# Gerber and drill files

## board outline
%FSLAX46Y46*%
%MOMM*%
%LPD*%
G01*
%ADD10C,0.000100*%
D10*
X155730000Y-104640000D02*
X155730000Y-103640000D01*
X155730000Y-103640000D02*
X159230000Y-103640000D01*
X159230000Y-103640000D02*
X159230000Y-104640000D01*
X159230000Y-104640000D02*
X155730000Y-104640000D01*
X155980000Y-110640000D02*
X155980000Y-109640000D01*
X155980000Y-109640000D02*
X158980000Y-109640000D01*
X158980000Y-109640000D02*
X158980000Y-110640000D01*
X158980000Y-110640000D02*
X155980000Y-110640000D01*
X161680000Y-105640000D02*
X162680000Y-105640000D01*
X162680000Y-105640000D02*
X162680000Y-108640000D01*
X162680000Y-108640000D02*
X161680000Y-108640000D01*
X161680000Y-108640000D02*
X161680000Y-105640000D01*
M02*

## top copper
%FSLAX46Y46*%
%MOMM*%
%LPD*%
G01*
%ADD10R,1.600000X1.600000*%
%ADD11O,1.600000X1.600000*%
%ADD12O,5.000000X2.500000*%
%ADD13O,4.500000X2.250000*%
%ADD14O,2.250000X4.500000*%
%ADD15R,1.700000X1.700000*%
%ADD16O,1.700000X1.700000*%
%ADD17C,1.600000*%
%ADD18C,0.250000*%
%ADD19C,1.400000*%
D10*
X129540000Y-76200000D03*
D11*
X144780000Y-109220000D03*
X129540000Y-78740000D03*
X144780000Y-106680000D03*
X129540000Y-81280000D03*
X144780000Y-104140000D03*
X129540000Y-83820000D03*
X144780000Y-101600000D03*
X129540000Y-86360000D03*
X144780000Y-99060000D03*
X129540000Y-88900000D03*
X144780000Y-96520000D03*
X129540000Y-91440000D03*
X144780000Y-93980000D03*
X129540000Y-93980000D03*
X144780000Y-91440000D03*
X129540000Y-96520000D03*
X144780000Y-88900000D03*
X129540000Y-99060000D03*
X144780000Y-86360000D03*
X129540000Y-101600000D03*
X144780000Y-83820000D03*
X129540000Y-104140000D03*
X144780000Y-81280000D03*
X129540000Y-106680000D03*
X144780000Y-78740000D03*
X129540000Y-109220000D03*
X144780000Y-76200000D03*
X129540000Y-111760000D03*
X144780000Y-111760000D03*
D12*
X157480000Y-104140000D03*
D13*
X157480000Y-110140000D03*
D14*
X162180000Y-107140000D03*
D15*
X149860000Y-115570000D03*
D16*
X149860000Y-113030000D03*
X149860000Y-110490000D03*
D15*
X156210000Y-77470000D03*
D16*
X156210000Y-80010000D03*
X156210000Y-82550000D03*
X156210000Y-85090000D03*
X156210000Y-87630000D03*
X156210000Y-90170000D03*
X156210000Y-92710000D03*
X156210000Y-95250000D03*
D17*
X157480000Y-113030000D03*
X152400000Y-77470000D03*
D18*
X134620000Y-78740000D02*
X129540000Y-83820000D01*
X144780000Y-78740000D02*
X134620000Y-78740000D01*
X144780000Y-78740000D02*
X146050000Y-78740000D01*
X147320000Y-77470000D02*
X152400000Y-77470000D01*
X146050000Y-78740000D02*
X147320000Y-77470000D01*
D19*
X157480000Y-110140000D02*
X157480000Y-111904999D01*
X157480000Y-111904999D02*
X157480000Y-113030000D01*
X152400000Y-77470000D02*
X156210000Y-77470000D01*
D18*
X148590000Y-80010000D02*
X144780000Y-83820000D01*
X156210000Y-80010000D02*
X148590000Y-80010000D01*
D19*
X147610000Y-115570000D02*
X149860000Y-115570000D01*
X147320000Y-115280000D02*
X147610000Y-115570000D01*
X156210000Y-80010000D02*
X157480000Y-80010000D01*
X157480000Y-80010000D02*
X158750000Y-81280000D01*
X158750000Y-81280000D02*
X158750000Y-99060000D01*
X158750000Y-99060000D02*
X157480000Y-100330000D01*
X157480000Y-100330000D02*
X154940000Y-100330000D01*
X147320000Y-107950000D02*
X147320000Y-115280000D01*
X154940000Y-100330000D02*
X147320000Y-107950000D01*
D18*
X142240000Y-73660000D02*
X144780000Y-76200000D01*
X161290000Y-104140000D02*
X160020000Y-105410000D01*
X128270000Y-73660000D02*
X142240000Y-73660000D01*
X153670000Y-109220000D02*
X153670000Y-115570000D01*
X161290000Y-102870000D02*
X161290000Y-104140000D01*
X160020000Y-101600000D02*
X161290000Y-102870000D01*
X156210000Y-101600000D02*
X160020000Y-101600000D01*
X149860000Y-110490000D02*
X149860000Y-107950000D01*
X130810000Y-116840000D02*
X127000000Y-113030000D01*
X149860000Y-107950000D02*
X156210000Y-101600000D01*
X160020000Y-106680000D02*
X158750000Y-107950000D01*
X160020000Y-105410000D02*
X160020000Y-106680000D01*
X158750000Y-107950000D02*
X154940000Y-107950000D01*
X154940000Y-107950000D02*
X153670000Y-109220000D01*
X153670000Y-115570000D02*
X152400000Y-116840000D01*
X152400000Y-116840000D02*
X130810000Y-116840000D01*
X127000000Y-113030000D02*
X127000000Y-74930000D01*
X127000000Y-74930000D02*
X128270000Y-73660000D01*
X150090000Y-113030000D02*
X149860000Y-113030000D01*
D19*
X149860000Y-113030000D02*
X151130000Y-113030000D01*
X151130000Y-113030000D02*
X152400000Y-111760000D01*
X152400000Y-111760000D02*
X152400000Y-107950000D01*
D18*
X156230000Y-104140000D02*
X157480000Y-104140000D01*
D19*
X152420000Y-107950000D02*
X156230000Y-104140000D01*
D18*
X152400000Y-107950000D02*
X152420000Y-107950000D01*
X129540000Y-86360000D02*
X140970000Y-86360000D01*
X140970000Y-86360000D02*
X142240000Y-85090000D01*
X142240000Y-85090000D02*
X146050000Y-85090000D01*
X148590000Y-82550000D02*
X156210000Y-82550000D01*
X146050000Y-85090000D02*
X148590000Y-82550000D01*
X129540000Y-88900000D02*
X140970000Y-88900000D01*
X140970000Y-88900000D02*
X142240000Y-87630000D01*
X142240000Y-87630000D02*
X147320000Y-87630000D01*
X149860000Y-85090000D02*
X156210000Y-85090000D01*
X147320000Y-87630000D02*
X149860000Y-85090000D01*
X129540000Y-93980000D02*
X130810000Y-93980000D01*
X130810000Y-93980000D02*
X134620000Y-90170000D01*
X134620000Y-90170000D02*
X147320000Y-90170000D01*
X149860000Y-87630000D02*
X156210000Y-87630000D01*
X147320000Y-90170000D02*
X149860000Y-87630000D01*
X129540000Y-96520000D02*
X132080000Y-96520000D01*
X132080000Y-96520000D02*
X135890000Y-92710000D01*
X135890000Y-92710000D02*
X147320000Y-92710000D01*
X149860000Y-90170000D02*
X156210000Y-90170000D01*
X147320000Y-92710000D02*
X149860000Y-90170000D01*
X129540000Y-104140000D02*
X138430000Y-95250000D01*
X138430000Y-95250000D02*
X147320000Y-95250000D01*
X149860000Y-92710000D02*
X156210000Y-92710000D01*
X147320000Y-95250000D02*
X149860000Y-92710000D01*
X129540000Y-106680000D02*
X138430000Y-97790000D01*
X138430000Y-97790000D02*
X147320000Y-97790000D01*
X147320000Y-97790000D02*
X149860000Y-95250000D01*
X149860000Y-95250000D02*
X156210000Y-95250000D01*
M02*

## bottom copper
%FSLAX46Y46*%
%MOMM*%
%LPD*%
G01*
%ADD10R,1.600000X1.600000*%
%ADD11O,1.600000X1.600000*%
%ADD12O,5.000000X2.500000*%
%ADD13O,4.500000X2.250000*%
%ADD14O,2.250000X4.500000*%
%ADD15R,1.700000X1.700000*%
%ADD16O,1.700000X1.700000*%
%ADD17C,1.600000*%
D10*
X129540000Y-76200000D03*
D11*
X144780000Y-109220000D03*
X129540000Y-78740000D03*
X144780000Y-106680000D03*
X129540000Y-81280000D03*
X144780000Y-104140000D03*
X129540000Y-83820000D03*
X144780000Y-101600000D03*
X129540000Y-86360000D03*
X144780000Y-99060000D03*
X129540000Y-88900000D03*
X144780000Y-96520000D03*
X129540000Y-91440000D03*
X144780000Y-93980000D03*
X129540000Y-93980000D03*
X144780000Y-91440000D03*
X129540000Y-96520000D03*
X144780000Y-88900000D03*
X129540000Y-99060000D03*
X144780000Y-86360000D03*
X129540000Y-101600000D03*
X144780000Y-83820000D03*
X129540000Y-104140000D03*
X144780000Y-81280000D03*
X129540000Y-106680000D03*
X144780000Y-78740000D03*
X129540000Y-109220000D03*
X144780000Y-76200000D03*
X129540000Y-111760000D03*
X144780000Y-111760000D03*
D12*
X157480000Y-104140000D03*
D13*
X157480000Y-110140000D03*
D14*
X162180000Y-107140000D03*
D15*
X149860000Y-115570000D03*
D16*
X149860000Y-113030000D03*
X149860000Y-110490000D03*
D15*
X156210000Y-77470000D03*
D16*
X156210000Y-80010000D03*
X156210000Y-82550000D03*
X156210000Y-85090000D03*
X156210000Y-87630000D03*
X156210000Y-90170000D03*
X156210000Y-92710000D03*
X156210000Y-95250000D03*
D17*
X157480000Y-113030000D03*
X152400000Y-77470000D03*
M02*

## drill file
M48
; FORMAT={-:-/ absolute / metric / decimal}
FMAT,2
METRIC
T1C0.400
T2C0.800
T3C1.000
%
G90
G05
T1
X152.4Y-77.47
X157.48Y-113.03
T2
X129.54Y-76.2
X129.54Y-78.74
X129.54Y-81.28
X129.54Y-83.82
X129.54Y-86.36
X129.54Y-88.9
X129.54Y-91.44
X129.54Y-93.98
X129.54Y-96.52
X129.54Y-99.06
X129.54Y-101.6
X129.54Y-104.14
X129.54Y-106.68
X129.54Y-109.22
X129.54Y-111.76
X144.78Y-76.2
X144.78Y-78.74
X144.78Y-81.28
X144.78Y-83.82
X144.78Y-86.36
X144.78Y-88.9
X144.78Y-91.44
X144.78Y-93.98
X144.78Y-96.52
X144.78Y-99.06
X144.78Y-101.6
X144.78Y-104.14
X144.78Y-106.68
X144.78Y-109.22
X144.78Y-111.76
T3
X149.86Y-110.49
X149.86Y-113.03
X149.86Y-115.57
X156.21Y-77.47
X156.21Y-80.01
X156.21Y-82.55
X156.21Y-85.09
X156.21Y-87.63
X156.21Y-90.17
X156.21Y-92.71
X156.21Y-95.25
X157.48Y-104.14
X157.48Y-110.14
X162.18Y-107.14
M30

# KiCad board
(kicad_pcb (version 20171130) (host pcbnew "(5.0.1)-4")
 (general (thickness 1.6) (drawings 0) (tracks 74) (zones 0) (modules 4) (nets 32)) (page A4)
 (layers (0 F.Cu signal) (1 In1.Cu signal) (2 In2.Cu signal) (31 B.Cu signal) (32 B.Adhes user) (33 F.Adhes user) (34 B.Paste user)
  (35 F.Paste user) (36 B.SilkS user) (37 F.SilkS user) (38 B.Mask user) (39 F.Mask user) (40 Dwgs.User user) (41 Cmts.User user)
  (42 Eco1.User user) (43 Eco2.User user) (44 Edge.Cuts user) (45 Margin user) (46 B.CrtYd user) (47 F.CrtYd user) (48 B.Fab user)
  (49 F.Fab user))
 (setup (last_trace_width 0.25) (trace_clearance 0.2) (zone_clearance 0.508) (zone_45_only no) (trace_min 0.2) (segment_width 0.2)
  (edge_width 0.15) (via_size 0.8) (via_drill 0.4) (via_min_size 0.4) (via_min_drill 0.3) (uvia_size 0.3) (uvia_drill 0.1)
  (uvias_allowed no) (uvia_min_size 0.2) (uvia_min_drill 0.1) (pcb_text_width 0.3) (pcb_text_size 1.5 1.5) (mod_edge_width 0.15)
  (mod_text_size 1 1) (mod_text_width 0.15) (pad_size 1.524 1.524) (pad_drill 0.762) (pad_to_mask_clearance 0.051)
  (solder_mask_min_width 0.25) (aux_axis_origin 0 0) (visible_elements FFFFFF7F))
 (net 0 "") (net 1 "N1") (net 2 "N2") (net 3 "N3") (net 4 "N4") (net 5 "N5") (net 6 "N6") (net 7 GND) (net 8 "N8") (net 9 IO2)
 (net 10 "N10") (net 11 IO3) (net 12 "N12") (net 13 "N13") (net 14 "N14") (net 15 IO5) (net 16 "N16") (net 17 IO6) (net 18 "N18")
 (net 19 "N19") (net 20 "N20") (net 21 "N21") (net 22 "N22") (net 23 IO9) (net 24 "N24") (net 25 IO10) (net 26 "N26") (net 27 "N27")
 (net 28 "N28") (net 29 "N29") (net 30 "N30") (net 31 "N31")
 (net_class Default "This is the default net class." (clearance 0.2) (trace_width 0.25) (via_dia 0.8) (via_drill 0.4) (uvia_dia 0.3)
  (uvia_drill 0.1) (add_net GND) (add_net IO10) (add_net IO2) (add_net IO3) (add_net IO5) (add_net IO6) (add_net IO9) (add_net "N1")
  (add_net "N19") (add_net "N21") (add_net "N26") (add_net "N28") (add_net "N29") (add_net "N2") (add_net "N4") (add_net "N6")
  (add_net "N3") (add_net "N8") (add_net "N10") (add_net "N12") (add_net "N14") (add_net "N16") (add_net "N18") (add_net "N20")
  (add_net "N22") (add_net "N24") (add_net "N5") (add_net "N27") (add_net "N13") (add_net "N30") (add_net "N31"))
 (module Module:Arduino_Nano (layer F.Cu) (at 129.54 76.2)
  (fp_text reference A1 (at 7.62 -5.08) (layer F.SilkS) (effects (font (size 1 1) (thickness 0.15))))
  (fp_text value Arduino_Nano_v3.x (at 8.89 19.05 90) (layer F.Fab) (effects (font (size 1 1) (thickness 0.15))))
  (pad 1 thru_hole rect (at 0 0) (size 1.6 1.6) (drill 0.8) (layers *.Cu *.Mask) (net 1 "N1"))
  (pad 17 thru_hole oval (at 15.24 33.02) (size 1.6 1.6) (drill 0.8) (layers *.Cu *.Mask) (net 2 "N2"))
  (pad 2 thru_hole oval (at 0 2.54) (size 1.6 1.6) (drill 0.8) (layers *.Cu *.Mask) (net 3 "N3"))
  (pad 18 thru_hole oval (at 15.24 30.48) (size 1.6 1.6) (drill 0.8) (layers *.Cu *.Mask) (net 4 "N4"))
  (pad 3 thru_hole oval (at 0 5.08) (size 1.6 1.6) (drill 0.8) (layers *.Cu *.Mask) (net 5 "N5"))
  (pad 19 thru_hole oval (at 15.24 27.94) (size 1.6 1.6) (drill 0.8) (layers *.Cu *.Mask) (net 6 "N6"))
  (pad 4 thru_hole oval (at 0 7.62) (size 1.6 1.6) (drill 0.8) (layers *.Cu *.Mask) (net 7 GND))
  (pad 20 thru_hole oval (at 15.24 25.4) (size 1.6 1.6) (drill 0.8) (layers *.Cu *.Mask) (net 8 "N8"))
  (pad 5 thru_hole oval (at 0 10.16) (size 1.6 1.6) (drill 0.8) (layers *.Cu *.Mask) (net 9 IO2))
  (pad 21 thru_hole oval (at 15.24 22.86) (size 1.6 1.6) (drill 0.8) (layers *.Cu *.Mask) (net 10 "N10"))
  (pad 6 thru_hole oval (at 0 12.7) (size 1.6 1.6) (drill 0.8) (layers *.Cu *.Mask) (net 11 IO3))
  (pad 22 thru_hole oval (at 15.24 20.32) (size 1.6 1.6) (drill 0.8) (layers *.Cu *.Mask) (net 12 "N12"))
  (pad 7 thru_hole oval (at 0 15.24) (size 1.6 1.6) (drill 0.8) (layers *.Cu *.Mask) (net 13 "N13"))
  (pad 23 thru_hole oval (at 15.24 17.78) (size 1.6 1.6) (drill 0.8) (layers *.Cu *.Mask) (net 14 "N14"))
  (pad 8 thru_hole oval (at 0 17.78) (size 1.6 1.6) (drill 0.8) (layers *.Cu *.Mask) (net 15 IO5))
  (pad 24 thru_hole oval (at 15.24 15.24) (size 1.6 1.6) (drill 0.8) (layers *.Cu *.Mask) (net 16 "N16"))
  (pad 9 thru_hole oval (at 0 20.32) (size 1.6 1.6) (drill 0.8) (layers *.Cu *.Mask) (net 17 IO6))
  (pad 25 thru_hole oval (at 15.24 12.7) (size 1.6 1.6) (drill 0.8) (layers *.Cu *.Mask) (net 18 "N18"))
  (pad 10 thru_hole oval (at 0 22.86) (size 1.6 1.6) (drill 0.8) (layers *.Cu *.Mask) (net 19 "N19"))
  (pad 26 thru_hole oval (at 15.24 10.16) (size 1.6 1.6) (drill 0.8) (layers *.Cu *.Mask) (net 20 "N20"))
  (pad 11 thru_hole oval (at 0 25.4) (size 1.6 1.6) (drill 0.8) (layers *.Cu *.Mask) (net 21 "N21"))
  (pad 27 thru_hole oval (at 15.24 7.62) (size 1.6 1.6) (drill 0.8) (layers *.Cu *.Mask) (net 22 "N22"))
  (pad 12 thru_hole oval (at 0 27.94) (size 1.6 1.6) (drill 0.8) (layers *.Cu *.Mask) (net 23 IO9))
  (pad 28 thru_hole oval (at 15.24 5.08) (size 1.6 1.6) (drill 0.8) (layers *.Cu *.Mask) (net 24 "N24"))
  (pad 13 thru_hole oval (at 0 30.48) (size 1.6 1.6) (drill 0.8) (layers *.Cu *.Mask) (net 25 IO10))
  (pad 29 thru_hole oval (at 15.24 2.54) (size 1.6 1.6) (drill 0.8) (layers *.Cu *.Mask) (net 7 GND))
  (pad 14 thru_hole oval (at 0 33.02) (size 1.6 1.6) (drill 0.8) (layers *.Cu *.Mask) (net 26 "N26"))
  (pad 30 thru_hole oval (at 15.24 0) (size 1.6 1.6) (drill 0.8) (layers *.Cu *.Mask) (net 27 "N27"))
  (pad 15 thru_hole oval (at 0 35.56) (size 1.6 1.6) (drill 0.8) (layers *.Cu *.Mask) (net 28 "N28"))
  (pad 16 thru_hole oval (at 15.24 35.56) (size 1.6 1.6) (drill 0.8) (layers *.Cu *.Mask) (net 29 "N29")))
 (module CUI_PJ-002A (layer F.Cu) (at 157.48 104.14 270)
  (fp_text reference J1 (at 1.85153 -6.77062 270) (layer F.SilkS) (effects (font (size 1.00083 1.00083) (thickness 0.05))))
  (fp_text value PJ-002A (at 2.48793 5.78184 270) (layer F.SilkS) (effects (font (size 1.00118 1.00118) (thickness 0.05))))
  (fp_line (start 0.5 1.75) (end -0.5 1.75) (layer Edge.Cuts) (width 0.0001))
  (fp_line (start -0.5 1.75) (end -0.5 -1.75) (layer Edge.Cuts) (width 0.0001))
  (fp_line (start -0.5 -1.75) (end 0.5 -1.75) (layer Edge.Cuts) (width 0.0001))
  (fp_line (start 0.5 -1.75) (end 0.5 1.75) (layer Edge.Cuts) (width 0.0001))
  (fp_line (start 6.5 1.5) (end 5.5 1.5) (layer Edge.Cuts) (width 0.0001))
  (fp_line (start 5.5 1.5) (end 5.5 -1.5) (layer Edge.Cuts) (width 0.0001))
  (fp_line (start 5.5 -1.5) (end 6.5 -1.5) (layer Edge.Cuts) (width 0.0001))
  (fp_line (start 6.5 -1.5) (end 6.5 1.5) (layer Edge.Cuts) (width 0.0001))
  (fp_line (start 1.5 -4.2) (end 1.5 -5.2) (layer Edge.Cuts) (width 0.0001))
  (fp_line (start 1.5 -5.2) (end 4.5 -5.2) (layer Edge.Cuts) (width 0.0001))
  (fp_line (start 4.5 -5.2) (end 4.5 -4.2) (layer Edge.Cuts) (width 0.0001))
  (fp_line (start 4.5 -4.2) (end 1.5 -4.2) (layer Edge.Cuts) (width 0.0001))
  (pad 1 thru_hole oval (at 0 0) (size 5 2.5) (drill 1) (layers *.Cu *.Mask) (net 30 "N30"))
  (pad 2 thru_hole oval (at 6 0) (size 4.5 2.25) (drill 1) (layers *.Cu *.Mask) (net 7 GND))
  (pad 3 thru_hole oval (at 3 -4.7 90) (size 4.5 2.25) (drill 1) (layers *.Cu *.Mask) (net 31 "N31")))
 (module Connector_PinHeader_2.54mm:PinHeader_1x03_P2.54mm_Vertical (layer F.Cu) (at 149.86 115.57 180)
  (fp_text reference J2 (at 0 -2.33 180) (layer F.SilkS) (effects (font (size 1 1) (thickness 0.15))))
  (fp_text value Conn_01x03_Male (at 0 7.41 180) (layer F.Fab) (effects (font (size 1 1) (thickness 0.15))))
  (pad 1 thru_hole rect (at 0 0 180) (size 1.7 1.7) (drill 1) (layers *.Cu *.Mask) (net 22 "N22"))
  (pad 2 thru_hole oval (at 0 2.54 180) (size 1.7 1.7) (drill 1) (layers *.Cu *.Mask) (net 30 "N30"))
  (pad 3 thru_hole oval (at 0 5.08 180) (size 1.7 1.7) (drill 1) (layers *.Cu *.Mask) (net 27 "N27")))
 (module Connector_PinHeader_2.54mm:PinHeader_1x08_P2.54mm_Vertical (layer F.Cu) (at 156.21 77.47)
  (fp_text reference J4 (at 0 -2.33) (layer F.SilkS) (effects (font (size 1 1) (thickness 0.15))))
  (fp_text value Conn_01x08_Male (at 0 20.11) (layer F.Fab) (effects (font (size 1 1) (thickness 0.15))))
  (pad 1 thru_hole rect (at 0 0) (size 1.7 1.7) (drill 1) (layers *.Cu *.Mask) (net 7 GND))
  (pad 2 thru_hole oval (at 0 2.54) (size 1.7 1.7) (drill 1) (layers *.Cu *.Mask) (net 22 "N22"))
  (pad 3 thru_hole oval (at 0 5.08) (size 1.7 1.7) (drill 1) (layers *.Cu *.Mask) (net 9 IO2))
  (pad 4 thru_hole oval (at 0 7.62) (size 1.7 1.7) (drill 1) (layers *.Cu *.Mask) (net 11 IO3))
  (pad 5 thru_hole oval (at 0 10.16) (size 1.7 1.7) (drill 1) (layers *.Cu *.Mask) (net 15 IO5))
  (pad 6 thru_hole oval (at 0 12.7) (size 1.7 1.7) (drill 1) (layers *.Cu *.Mask) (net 17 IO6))
  (pad 7 thru_hole oval (at 0 15.24) (size 1.7 1.7) (drill 1) (layers *.Cu *.Mask) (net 23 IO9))
  (pad 8 thru_hole oval (at 0 17.78) (size 1.7 1.7) (drill 1) (layers *.Cu *.Mask) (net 25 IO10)))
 (via (at 157.48 113.03) (size 1.6) (drill 0.4) (layers F.Cu B.Cu) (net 7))
 (segment (start 134.62 78.74) (end 129.54 83.82) (width 0.25) (layer F.Cu) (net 7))
 (segment (start 144.78 78.74) (end 134.62 78.74) (width 0.25) (layer F.Cu) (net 7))
 (segment (start 144.78 78.74) (end 146.05 78.74) (width 0.25) (layer F.Cu) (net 7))
 (segment (start 147.32 77.47) (end 152.4 77.47) (width 0.25) (layer F.Cu) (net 7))
 (segment (start 146.05 78.74) (end 147.32 77.47) (width 0.25) (layer F.Cu) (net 7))
 (segment (start 157.48 110.14) (end 157.48 111.904999) (width 1.4) (layer F.Cu) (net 7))
 (segment (start 157.48 111.904999) (end 157.48 113.03) (width 1.4) (layer F.Cu) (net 7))
 (segment (start 152.4 77.47) (end 156.21 77.47) (width 1.4) (layer F.Cu) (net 7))
 (via (at 152.4 77.47) (size 1.6) (drill 0.4) (layers F.Cu B.Cu) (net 7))
 (segment (start 148.59 80.01) (end 144.78 83.82) (width 0.25) (layer F.Cu) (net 22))
 (segment (start 156.21 80.01) (end 148.59 80.01) (width 0.25) (layer F.Cu) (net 22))
 (segment (start 147.61 115.57) (end 149.86 115.57) (width 1.4) (layer F.Cu) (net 22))
 (segment (start 147.32 115.28) (end 147.61 115.57) (width 1.4) (layer F.Cu) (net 22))
 (segment (start 156.21 80.01) (end 157.48 80.01) (width 1.4) (layer F.Cu) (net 22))
 (segment (start 157.48 80.01) (end 158.75 81.28) (width 1.4) (layer F.Cu) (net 22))
 (segment (start 158.75 81.28) (end 158.75 99.06) (width 1.4) (layer F.Cu) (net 22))
 (segment (start 158.75 99.06) (end 157.48 100.33) (width 1.4) (layer F.Cu) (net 22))
 (segment (start 157.48 100.33) (end 154.94 100.33) (width 1.4) (layer F.Cu) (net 22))
 (segment (start 147.32 107.95) (end 147.32 115.28) (width 1.4) (layer F.Cu) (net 22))
 (segment (start 154.94 100.33) (end 147.32 107.95) (width 1.4) (layer F.Cu) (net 22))
 (segment (start 142.24 73.66) (end 144.78 76.2) (width 0.25) (layer F.Cu) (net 27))
 (segment (start 161.29 104.14) (end 160.02 105.41) (width 0.25) (layer F.Cu) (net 27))
 (segment (start 128.27 73.66) (end 142.24 73.66) (width 0.25) (layer F.Cu) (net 27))
 (segment (start 153.67 109.22) (end 153.67 115.57) (width 0.25) (layer F.Cu) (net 27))
 (segment (start 161.29 102.87) (end 161.29 104.14) (width 0.25) (layer F.Cu) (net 27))
 (segment (start 160.02 101.6) (end 161.29 102.87) (width 0.25) (layer F.Cu) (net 27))
 (segment (start 156.21 101.6) (end 160.02 101.6) (width 0.25) (layer F.Cu) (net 27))
 (segment (start 149.86 110.49) (end 149.86 107.95) (width 0.25) (layer F.Cu) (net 27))
 (segment (start 130.81 116.84) (end 127 113.03) (width 0.25) (layer F.Cu) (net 27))
 (segment (start 149.86 107.95) (end 156.21 101.6) (width 0.25) (layer F.Cu) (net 27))
 (segment (start 160.02 106.68) (end 158.75 107.95) (width 0.25) (layer F.Cu) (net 27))
 (segment (start 160.02 105.41) (end 160.02 106.68) (width 0.25) (layer F.Cu) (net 27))
 (segment (start 158.75 107.95) (end 154.94 107.95) (width 0.25) (layer F.Cu) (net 27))
 (segment (start 154.94 107.95) (end 153.67 109.22) (width 0.25) (layer F.Cu) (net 27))
 (segment (start 153.67 115.57) (end 152.4 116.84) (width 0.25) (layer F.Cu) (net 27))
 (segment (start 152.4 116.84) (end 130.81 116.84) (width 0.25) (layer F.Cu) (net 27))
 (segment (start 127 113.03) (end 127 74.93) (width 0.25) (layer F.Cu) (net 27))
 (segment (start 127 74.93) (end 128.27 73.66) (width 0.25) (layer F.Cu) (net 27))
 (segment (start 150.09 113.03) (end 149.86 113.03) (width 0.25) (layer F.Cu) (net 30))
 (segment (start 149.86 113.03) (end 151.13 113.03) (width 1.4) (layer F.Cu) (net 30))
 (segment (start 151.13 113.03) (end 152.4 111.76) (width 1.4) (layer F.Cu) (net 30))
 (segment (start 152.4 111.76) (end 152.4 107.95) (width 1.4) (layer F.Cu) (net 30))
 (segment (start 156.23 104.14) (end 157.48 104.14) (width 0.25) (layer F.Cu) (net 30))
 (segment (start 152.42 107.95) (end 156.23 104.14) (width 1.4) (layer F.Cu) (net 30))
 (segment (start 152.4 107.95) (end 152.42 107.95) (width 0.25) (layer F.Cu) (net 30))
 (segment (start 129.54 86.36) (end 140.97 86.36) (width 0.25) (layer F.Cu) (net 9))
 (segment (start 140.97 86.36) (end 142.24 85.09) (width 0.25) (layer F.Cu) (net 9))
 (segment (start 142.24 85.09) (end 146.05 85.09) (width 0.25) (layer F.Cu) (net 9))
 (segment (start 148.59 82.55) (end 156.21 82.55) (width 0.25) (layer F.Cu) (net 9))
 (segment (start 146.05 85.09) (end 148.59 82.55) (width 0.25) (layer F.Cu) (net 9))
 (segment (start 129.54 88.9) (end 140.97 88.9) (width 0.25) (layer F.Cu) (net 11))
 (segment (start 140.97 88.9) (end 142.24 87.63) (width 0.25) (layer F.Cu) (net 11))
 (segment (start 142.24 87.63) (end 147.32 87.63) (width 0.25) (layer F.Cu) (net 11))
 (segment (start 149.86 85.09) (end 156.21 85.09) (width 0.25) (layer F.Cu) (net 11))
 (segment (start 147.32 87.63) (end 149.86 85.09) (width 0.25) (layer F.Cu) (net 11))
 (segment (start 129.54 93.98) (end 130.81 93.98) (width 0.25) (layer F.Cu) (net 15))
 (segment (start 130.81 93.98) (end 134.62 90.17) (width 0.25) (layer F.Cu) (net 15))
 (segment (start 134.62 90.17) (end 147.32 90.17) (width 0.25) (layer F.Cu) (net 15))
 (segment (start 149.86 87.63) (end 156.21 87.63) (width 0.25) (layer F.Cu) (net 15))
 (segment (start 147.32 90.17) (end 149.86 87.63) (width 0.25) (layer F.Cu) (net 15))
 (segment (start 129.54 96.52) (end 132.08 96.52) (width 0.25) (layer F.Cu) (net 17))
 (segment (start 132.08 96.52) (end 135.89 92.71) (width 0.25) (layer F.Cu) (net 17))
 (segment (start 135.89 92.71) (end 147.32 92.71) (width 0.25) (layer F.Cu) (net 17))
 (segment (start 149.86 90.17) (end 156.21 90.17) (width 0.25) (layer F.Cu) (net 17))
 (segment (start 147.32 92.71) (end 149.86 90.17) (width 0.25) (layer F.Cu) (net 17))
 (segment (start 129.54 104.14) (end 138.43 95.25) (width 0.25) (layer F.Cu) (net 23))
 (segment (start 138.43 95.25) (end 147.32 95.25) (width 0.25) (layer F.Cu) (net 23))
 (segment (start 149.86 92.71) (end 156.21 92.71) (width 0.25) (layer F.Cu) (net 23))
 (segment (start 147.32 95.25) (end 149.86 92.71) (width 0.25) (layer F.Cu) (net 23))
 (segment (start 129.54 106.68) (end 138.43 97.79) (width 0.25) (layer F.Cu) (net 25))
 (segment (start 138.43 97.79) (end 147.32 97.79) (width 0.25) (layer F.Cu) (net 25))
 (segment (start 147.32 97.79) (end 149.86 95.25) (width 0.25) (layer F.Cu) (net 25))
 (segment (start 149.86 95.25) (end 156.21 95.25) (width 0.25) (layer F.Cu) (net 25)))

